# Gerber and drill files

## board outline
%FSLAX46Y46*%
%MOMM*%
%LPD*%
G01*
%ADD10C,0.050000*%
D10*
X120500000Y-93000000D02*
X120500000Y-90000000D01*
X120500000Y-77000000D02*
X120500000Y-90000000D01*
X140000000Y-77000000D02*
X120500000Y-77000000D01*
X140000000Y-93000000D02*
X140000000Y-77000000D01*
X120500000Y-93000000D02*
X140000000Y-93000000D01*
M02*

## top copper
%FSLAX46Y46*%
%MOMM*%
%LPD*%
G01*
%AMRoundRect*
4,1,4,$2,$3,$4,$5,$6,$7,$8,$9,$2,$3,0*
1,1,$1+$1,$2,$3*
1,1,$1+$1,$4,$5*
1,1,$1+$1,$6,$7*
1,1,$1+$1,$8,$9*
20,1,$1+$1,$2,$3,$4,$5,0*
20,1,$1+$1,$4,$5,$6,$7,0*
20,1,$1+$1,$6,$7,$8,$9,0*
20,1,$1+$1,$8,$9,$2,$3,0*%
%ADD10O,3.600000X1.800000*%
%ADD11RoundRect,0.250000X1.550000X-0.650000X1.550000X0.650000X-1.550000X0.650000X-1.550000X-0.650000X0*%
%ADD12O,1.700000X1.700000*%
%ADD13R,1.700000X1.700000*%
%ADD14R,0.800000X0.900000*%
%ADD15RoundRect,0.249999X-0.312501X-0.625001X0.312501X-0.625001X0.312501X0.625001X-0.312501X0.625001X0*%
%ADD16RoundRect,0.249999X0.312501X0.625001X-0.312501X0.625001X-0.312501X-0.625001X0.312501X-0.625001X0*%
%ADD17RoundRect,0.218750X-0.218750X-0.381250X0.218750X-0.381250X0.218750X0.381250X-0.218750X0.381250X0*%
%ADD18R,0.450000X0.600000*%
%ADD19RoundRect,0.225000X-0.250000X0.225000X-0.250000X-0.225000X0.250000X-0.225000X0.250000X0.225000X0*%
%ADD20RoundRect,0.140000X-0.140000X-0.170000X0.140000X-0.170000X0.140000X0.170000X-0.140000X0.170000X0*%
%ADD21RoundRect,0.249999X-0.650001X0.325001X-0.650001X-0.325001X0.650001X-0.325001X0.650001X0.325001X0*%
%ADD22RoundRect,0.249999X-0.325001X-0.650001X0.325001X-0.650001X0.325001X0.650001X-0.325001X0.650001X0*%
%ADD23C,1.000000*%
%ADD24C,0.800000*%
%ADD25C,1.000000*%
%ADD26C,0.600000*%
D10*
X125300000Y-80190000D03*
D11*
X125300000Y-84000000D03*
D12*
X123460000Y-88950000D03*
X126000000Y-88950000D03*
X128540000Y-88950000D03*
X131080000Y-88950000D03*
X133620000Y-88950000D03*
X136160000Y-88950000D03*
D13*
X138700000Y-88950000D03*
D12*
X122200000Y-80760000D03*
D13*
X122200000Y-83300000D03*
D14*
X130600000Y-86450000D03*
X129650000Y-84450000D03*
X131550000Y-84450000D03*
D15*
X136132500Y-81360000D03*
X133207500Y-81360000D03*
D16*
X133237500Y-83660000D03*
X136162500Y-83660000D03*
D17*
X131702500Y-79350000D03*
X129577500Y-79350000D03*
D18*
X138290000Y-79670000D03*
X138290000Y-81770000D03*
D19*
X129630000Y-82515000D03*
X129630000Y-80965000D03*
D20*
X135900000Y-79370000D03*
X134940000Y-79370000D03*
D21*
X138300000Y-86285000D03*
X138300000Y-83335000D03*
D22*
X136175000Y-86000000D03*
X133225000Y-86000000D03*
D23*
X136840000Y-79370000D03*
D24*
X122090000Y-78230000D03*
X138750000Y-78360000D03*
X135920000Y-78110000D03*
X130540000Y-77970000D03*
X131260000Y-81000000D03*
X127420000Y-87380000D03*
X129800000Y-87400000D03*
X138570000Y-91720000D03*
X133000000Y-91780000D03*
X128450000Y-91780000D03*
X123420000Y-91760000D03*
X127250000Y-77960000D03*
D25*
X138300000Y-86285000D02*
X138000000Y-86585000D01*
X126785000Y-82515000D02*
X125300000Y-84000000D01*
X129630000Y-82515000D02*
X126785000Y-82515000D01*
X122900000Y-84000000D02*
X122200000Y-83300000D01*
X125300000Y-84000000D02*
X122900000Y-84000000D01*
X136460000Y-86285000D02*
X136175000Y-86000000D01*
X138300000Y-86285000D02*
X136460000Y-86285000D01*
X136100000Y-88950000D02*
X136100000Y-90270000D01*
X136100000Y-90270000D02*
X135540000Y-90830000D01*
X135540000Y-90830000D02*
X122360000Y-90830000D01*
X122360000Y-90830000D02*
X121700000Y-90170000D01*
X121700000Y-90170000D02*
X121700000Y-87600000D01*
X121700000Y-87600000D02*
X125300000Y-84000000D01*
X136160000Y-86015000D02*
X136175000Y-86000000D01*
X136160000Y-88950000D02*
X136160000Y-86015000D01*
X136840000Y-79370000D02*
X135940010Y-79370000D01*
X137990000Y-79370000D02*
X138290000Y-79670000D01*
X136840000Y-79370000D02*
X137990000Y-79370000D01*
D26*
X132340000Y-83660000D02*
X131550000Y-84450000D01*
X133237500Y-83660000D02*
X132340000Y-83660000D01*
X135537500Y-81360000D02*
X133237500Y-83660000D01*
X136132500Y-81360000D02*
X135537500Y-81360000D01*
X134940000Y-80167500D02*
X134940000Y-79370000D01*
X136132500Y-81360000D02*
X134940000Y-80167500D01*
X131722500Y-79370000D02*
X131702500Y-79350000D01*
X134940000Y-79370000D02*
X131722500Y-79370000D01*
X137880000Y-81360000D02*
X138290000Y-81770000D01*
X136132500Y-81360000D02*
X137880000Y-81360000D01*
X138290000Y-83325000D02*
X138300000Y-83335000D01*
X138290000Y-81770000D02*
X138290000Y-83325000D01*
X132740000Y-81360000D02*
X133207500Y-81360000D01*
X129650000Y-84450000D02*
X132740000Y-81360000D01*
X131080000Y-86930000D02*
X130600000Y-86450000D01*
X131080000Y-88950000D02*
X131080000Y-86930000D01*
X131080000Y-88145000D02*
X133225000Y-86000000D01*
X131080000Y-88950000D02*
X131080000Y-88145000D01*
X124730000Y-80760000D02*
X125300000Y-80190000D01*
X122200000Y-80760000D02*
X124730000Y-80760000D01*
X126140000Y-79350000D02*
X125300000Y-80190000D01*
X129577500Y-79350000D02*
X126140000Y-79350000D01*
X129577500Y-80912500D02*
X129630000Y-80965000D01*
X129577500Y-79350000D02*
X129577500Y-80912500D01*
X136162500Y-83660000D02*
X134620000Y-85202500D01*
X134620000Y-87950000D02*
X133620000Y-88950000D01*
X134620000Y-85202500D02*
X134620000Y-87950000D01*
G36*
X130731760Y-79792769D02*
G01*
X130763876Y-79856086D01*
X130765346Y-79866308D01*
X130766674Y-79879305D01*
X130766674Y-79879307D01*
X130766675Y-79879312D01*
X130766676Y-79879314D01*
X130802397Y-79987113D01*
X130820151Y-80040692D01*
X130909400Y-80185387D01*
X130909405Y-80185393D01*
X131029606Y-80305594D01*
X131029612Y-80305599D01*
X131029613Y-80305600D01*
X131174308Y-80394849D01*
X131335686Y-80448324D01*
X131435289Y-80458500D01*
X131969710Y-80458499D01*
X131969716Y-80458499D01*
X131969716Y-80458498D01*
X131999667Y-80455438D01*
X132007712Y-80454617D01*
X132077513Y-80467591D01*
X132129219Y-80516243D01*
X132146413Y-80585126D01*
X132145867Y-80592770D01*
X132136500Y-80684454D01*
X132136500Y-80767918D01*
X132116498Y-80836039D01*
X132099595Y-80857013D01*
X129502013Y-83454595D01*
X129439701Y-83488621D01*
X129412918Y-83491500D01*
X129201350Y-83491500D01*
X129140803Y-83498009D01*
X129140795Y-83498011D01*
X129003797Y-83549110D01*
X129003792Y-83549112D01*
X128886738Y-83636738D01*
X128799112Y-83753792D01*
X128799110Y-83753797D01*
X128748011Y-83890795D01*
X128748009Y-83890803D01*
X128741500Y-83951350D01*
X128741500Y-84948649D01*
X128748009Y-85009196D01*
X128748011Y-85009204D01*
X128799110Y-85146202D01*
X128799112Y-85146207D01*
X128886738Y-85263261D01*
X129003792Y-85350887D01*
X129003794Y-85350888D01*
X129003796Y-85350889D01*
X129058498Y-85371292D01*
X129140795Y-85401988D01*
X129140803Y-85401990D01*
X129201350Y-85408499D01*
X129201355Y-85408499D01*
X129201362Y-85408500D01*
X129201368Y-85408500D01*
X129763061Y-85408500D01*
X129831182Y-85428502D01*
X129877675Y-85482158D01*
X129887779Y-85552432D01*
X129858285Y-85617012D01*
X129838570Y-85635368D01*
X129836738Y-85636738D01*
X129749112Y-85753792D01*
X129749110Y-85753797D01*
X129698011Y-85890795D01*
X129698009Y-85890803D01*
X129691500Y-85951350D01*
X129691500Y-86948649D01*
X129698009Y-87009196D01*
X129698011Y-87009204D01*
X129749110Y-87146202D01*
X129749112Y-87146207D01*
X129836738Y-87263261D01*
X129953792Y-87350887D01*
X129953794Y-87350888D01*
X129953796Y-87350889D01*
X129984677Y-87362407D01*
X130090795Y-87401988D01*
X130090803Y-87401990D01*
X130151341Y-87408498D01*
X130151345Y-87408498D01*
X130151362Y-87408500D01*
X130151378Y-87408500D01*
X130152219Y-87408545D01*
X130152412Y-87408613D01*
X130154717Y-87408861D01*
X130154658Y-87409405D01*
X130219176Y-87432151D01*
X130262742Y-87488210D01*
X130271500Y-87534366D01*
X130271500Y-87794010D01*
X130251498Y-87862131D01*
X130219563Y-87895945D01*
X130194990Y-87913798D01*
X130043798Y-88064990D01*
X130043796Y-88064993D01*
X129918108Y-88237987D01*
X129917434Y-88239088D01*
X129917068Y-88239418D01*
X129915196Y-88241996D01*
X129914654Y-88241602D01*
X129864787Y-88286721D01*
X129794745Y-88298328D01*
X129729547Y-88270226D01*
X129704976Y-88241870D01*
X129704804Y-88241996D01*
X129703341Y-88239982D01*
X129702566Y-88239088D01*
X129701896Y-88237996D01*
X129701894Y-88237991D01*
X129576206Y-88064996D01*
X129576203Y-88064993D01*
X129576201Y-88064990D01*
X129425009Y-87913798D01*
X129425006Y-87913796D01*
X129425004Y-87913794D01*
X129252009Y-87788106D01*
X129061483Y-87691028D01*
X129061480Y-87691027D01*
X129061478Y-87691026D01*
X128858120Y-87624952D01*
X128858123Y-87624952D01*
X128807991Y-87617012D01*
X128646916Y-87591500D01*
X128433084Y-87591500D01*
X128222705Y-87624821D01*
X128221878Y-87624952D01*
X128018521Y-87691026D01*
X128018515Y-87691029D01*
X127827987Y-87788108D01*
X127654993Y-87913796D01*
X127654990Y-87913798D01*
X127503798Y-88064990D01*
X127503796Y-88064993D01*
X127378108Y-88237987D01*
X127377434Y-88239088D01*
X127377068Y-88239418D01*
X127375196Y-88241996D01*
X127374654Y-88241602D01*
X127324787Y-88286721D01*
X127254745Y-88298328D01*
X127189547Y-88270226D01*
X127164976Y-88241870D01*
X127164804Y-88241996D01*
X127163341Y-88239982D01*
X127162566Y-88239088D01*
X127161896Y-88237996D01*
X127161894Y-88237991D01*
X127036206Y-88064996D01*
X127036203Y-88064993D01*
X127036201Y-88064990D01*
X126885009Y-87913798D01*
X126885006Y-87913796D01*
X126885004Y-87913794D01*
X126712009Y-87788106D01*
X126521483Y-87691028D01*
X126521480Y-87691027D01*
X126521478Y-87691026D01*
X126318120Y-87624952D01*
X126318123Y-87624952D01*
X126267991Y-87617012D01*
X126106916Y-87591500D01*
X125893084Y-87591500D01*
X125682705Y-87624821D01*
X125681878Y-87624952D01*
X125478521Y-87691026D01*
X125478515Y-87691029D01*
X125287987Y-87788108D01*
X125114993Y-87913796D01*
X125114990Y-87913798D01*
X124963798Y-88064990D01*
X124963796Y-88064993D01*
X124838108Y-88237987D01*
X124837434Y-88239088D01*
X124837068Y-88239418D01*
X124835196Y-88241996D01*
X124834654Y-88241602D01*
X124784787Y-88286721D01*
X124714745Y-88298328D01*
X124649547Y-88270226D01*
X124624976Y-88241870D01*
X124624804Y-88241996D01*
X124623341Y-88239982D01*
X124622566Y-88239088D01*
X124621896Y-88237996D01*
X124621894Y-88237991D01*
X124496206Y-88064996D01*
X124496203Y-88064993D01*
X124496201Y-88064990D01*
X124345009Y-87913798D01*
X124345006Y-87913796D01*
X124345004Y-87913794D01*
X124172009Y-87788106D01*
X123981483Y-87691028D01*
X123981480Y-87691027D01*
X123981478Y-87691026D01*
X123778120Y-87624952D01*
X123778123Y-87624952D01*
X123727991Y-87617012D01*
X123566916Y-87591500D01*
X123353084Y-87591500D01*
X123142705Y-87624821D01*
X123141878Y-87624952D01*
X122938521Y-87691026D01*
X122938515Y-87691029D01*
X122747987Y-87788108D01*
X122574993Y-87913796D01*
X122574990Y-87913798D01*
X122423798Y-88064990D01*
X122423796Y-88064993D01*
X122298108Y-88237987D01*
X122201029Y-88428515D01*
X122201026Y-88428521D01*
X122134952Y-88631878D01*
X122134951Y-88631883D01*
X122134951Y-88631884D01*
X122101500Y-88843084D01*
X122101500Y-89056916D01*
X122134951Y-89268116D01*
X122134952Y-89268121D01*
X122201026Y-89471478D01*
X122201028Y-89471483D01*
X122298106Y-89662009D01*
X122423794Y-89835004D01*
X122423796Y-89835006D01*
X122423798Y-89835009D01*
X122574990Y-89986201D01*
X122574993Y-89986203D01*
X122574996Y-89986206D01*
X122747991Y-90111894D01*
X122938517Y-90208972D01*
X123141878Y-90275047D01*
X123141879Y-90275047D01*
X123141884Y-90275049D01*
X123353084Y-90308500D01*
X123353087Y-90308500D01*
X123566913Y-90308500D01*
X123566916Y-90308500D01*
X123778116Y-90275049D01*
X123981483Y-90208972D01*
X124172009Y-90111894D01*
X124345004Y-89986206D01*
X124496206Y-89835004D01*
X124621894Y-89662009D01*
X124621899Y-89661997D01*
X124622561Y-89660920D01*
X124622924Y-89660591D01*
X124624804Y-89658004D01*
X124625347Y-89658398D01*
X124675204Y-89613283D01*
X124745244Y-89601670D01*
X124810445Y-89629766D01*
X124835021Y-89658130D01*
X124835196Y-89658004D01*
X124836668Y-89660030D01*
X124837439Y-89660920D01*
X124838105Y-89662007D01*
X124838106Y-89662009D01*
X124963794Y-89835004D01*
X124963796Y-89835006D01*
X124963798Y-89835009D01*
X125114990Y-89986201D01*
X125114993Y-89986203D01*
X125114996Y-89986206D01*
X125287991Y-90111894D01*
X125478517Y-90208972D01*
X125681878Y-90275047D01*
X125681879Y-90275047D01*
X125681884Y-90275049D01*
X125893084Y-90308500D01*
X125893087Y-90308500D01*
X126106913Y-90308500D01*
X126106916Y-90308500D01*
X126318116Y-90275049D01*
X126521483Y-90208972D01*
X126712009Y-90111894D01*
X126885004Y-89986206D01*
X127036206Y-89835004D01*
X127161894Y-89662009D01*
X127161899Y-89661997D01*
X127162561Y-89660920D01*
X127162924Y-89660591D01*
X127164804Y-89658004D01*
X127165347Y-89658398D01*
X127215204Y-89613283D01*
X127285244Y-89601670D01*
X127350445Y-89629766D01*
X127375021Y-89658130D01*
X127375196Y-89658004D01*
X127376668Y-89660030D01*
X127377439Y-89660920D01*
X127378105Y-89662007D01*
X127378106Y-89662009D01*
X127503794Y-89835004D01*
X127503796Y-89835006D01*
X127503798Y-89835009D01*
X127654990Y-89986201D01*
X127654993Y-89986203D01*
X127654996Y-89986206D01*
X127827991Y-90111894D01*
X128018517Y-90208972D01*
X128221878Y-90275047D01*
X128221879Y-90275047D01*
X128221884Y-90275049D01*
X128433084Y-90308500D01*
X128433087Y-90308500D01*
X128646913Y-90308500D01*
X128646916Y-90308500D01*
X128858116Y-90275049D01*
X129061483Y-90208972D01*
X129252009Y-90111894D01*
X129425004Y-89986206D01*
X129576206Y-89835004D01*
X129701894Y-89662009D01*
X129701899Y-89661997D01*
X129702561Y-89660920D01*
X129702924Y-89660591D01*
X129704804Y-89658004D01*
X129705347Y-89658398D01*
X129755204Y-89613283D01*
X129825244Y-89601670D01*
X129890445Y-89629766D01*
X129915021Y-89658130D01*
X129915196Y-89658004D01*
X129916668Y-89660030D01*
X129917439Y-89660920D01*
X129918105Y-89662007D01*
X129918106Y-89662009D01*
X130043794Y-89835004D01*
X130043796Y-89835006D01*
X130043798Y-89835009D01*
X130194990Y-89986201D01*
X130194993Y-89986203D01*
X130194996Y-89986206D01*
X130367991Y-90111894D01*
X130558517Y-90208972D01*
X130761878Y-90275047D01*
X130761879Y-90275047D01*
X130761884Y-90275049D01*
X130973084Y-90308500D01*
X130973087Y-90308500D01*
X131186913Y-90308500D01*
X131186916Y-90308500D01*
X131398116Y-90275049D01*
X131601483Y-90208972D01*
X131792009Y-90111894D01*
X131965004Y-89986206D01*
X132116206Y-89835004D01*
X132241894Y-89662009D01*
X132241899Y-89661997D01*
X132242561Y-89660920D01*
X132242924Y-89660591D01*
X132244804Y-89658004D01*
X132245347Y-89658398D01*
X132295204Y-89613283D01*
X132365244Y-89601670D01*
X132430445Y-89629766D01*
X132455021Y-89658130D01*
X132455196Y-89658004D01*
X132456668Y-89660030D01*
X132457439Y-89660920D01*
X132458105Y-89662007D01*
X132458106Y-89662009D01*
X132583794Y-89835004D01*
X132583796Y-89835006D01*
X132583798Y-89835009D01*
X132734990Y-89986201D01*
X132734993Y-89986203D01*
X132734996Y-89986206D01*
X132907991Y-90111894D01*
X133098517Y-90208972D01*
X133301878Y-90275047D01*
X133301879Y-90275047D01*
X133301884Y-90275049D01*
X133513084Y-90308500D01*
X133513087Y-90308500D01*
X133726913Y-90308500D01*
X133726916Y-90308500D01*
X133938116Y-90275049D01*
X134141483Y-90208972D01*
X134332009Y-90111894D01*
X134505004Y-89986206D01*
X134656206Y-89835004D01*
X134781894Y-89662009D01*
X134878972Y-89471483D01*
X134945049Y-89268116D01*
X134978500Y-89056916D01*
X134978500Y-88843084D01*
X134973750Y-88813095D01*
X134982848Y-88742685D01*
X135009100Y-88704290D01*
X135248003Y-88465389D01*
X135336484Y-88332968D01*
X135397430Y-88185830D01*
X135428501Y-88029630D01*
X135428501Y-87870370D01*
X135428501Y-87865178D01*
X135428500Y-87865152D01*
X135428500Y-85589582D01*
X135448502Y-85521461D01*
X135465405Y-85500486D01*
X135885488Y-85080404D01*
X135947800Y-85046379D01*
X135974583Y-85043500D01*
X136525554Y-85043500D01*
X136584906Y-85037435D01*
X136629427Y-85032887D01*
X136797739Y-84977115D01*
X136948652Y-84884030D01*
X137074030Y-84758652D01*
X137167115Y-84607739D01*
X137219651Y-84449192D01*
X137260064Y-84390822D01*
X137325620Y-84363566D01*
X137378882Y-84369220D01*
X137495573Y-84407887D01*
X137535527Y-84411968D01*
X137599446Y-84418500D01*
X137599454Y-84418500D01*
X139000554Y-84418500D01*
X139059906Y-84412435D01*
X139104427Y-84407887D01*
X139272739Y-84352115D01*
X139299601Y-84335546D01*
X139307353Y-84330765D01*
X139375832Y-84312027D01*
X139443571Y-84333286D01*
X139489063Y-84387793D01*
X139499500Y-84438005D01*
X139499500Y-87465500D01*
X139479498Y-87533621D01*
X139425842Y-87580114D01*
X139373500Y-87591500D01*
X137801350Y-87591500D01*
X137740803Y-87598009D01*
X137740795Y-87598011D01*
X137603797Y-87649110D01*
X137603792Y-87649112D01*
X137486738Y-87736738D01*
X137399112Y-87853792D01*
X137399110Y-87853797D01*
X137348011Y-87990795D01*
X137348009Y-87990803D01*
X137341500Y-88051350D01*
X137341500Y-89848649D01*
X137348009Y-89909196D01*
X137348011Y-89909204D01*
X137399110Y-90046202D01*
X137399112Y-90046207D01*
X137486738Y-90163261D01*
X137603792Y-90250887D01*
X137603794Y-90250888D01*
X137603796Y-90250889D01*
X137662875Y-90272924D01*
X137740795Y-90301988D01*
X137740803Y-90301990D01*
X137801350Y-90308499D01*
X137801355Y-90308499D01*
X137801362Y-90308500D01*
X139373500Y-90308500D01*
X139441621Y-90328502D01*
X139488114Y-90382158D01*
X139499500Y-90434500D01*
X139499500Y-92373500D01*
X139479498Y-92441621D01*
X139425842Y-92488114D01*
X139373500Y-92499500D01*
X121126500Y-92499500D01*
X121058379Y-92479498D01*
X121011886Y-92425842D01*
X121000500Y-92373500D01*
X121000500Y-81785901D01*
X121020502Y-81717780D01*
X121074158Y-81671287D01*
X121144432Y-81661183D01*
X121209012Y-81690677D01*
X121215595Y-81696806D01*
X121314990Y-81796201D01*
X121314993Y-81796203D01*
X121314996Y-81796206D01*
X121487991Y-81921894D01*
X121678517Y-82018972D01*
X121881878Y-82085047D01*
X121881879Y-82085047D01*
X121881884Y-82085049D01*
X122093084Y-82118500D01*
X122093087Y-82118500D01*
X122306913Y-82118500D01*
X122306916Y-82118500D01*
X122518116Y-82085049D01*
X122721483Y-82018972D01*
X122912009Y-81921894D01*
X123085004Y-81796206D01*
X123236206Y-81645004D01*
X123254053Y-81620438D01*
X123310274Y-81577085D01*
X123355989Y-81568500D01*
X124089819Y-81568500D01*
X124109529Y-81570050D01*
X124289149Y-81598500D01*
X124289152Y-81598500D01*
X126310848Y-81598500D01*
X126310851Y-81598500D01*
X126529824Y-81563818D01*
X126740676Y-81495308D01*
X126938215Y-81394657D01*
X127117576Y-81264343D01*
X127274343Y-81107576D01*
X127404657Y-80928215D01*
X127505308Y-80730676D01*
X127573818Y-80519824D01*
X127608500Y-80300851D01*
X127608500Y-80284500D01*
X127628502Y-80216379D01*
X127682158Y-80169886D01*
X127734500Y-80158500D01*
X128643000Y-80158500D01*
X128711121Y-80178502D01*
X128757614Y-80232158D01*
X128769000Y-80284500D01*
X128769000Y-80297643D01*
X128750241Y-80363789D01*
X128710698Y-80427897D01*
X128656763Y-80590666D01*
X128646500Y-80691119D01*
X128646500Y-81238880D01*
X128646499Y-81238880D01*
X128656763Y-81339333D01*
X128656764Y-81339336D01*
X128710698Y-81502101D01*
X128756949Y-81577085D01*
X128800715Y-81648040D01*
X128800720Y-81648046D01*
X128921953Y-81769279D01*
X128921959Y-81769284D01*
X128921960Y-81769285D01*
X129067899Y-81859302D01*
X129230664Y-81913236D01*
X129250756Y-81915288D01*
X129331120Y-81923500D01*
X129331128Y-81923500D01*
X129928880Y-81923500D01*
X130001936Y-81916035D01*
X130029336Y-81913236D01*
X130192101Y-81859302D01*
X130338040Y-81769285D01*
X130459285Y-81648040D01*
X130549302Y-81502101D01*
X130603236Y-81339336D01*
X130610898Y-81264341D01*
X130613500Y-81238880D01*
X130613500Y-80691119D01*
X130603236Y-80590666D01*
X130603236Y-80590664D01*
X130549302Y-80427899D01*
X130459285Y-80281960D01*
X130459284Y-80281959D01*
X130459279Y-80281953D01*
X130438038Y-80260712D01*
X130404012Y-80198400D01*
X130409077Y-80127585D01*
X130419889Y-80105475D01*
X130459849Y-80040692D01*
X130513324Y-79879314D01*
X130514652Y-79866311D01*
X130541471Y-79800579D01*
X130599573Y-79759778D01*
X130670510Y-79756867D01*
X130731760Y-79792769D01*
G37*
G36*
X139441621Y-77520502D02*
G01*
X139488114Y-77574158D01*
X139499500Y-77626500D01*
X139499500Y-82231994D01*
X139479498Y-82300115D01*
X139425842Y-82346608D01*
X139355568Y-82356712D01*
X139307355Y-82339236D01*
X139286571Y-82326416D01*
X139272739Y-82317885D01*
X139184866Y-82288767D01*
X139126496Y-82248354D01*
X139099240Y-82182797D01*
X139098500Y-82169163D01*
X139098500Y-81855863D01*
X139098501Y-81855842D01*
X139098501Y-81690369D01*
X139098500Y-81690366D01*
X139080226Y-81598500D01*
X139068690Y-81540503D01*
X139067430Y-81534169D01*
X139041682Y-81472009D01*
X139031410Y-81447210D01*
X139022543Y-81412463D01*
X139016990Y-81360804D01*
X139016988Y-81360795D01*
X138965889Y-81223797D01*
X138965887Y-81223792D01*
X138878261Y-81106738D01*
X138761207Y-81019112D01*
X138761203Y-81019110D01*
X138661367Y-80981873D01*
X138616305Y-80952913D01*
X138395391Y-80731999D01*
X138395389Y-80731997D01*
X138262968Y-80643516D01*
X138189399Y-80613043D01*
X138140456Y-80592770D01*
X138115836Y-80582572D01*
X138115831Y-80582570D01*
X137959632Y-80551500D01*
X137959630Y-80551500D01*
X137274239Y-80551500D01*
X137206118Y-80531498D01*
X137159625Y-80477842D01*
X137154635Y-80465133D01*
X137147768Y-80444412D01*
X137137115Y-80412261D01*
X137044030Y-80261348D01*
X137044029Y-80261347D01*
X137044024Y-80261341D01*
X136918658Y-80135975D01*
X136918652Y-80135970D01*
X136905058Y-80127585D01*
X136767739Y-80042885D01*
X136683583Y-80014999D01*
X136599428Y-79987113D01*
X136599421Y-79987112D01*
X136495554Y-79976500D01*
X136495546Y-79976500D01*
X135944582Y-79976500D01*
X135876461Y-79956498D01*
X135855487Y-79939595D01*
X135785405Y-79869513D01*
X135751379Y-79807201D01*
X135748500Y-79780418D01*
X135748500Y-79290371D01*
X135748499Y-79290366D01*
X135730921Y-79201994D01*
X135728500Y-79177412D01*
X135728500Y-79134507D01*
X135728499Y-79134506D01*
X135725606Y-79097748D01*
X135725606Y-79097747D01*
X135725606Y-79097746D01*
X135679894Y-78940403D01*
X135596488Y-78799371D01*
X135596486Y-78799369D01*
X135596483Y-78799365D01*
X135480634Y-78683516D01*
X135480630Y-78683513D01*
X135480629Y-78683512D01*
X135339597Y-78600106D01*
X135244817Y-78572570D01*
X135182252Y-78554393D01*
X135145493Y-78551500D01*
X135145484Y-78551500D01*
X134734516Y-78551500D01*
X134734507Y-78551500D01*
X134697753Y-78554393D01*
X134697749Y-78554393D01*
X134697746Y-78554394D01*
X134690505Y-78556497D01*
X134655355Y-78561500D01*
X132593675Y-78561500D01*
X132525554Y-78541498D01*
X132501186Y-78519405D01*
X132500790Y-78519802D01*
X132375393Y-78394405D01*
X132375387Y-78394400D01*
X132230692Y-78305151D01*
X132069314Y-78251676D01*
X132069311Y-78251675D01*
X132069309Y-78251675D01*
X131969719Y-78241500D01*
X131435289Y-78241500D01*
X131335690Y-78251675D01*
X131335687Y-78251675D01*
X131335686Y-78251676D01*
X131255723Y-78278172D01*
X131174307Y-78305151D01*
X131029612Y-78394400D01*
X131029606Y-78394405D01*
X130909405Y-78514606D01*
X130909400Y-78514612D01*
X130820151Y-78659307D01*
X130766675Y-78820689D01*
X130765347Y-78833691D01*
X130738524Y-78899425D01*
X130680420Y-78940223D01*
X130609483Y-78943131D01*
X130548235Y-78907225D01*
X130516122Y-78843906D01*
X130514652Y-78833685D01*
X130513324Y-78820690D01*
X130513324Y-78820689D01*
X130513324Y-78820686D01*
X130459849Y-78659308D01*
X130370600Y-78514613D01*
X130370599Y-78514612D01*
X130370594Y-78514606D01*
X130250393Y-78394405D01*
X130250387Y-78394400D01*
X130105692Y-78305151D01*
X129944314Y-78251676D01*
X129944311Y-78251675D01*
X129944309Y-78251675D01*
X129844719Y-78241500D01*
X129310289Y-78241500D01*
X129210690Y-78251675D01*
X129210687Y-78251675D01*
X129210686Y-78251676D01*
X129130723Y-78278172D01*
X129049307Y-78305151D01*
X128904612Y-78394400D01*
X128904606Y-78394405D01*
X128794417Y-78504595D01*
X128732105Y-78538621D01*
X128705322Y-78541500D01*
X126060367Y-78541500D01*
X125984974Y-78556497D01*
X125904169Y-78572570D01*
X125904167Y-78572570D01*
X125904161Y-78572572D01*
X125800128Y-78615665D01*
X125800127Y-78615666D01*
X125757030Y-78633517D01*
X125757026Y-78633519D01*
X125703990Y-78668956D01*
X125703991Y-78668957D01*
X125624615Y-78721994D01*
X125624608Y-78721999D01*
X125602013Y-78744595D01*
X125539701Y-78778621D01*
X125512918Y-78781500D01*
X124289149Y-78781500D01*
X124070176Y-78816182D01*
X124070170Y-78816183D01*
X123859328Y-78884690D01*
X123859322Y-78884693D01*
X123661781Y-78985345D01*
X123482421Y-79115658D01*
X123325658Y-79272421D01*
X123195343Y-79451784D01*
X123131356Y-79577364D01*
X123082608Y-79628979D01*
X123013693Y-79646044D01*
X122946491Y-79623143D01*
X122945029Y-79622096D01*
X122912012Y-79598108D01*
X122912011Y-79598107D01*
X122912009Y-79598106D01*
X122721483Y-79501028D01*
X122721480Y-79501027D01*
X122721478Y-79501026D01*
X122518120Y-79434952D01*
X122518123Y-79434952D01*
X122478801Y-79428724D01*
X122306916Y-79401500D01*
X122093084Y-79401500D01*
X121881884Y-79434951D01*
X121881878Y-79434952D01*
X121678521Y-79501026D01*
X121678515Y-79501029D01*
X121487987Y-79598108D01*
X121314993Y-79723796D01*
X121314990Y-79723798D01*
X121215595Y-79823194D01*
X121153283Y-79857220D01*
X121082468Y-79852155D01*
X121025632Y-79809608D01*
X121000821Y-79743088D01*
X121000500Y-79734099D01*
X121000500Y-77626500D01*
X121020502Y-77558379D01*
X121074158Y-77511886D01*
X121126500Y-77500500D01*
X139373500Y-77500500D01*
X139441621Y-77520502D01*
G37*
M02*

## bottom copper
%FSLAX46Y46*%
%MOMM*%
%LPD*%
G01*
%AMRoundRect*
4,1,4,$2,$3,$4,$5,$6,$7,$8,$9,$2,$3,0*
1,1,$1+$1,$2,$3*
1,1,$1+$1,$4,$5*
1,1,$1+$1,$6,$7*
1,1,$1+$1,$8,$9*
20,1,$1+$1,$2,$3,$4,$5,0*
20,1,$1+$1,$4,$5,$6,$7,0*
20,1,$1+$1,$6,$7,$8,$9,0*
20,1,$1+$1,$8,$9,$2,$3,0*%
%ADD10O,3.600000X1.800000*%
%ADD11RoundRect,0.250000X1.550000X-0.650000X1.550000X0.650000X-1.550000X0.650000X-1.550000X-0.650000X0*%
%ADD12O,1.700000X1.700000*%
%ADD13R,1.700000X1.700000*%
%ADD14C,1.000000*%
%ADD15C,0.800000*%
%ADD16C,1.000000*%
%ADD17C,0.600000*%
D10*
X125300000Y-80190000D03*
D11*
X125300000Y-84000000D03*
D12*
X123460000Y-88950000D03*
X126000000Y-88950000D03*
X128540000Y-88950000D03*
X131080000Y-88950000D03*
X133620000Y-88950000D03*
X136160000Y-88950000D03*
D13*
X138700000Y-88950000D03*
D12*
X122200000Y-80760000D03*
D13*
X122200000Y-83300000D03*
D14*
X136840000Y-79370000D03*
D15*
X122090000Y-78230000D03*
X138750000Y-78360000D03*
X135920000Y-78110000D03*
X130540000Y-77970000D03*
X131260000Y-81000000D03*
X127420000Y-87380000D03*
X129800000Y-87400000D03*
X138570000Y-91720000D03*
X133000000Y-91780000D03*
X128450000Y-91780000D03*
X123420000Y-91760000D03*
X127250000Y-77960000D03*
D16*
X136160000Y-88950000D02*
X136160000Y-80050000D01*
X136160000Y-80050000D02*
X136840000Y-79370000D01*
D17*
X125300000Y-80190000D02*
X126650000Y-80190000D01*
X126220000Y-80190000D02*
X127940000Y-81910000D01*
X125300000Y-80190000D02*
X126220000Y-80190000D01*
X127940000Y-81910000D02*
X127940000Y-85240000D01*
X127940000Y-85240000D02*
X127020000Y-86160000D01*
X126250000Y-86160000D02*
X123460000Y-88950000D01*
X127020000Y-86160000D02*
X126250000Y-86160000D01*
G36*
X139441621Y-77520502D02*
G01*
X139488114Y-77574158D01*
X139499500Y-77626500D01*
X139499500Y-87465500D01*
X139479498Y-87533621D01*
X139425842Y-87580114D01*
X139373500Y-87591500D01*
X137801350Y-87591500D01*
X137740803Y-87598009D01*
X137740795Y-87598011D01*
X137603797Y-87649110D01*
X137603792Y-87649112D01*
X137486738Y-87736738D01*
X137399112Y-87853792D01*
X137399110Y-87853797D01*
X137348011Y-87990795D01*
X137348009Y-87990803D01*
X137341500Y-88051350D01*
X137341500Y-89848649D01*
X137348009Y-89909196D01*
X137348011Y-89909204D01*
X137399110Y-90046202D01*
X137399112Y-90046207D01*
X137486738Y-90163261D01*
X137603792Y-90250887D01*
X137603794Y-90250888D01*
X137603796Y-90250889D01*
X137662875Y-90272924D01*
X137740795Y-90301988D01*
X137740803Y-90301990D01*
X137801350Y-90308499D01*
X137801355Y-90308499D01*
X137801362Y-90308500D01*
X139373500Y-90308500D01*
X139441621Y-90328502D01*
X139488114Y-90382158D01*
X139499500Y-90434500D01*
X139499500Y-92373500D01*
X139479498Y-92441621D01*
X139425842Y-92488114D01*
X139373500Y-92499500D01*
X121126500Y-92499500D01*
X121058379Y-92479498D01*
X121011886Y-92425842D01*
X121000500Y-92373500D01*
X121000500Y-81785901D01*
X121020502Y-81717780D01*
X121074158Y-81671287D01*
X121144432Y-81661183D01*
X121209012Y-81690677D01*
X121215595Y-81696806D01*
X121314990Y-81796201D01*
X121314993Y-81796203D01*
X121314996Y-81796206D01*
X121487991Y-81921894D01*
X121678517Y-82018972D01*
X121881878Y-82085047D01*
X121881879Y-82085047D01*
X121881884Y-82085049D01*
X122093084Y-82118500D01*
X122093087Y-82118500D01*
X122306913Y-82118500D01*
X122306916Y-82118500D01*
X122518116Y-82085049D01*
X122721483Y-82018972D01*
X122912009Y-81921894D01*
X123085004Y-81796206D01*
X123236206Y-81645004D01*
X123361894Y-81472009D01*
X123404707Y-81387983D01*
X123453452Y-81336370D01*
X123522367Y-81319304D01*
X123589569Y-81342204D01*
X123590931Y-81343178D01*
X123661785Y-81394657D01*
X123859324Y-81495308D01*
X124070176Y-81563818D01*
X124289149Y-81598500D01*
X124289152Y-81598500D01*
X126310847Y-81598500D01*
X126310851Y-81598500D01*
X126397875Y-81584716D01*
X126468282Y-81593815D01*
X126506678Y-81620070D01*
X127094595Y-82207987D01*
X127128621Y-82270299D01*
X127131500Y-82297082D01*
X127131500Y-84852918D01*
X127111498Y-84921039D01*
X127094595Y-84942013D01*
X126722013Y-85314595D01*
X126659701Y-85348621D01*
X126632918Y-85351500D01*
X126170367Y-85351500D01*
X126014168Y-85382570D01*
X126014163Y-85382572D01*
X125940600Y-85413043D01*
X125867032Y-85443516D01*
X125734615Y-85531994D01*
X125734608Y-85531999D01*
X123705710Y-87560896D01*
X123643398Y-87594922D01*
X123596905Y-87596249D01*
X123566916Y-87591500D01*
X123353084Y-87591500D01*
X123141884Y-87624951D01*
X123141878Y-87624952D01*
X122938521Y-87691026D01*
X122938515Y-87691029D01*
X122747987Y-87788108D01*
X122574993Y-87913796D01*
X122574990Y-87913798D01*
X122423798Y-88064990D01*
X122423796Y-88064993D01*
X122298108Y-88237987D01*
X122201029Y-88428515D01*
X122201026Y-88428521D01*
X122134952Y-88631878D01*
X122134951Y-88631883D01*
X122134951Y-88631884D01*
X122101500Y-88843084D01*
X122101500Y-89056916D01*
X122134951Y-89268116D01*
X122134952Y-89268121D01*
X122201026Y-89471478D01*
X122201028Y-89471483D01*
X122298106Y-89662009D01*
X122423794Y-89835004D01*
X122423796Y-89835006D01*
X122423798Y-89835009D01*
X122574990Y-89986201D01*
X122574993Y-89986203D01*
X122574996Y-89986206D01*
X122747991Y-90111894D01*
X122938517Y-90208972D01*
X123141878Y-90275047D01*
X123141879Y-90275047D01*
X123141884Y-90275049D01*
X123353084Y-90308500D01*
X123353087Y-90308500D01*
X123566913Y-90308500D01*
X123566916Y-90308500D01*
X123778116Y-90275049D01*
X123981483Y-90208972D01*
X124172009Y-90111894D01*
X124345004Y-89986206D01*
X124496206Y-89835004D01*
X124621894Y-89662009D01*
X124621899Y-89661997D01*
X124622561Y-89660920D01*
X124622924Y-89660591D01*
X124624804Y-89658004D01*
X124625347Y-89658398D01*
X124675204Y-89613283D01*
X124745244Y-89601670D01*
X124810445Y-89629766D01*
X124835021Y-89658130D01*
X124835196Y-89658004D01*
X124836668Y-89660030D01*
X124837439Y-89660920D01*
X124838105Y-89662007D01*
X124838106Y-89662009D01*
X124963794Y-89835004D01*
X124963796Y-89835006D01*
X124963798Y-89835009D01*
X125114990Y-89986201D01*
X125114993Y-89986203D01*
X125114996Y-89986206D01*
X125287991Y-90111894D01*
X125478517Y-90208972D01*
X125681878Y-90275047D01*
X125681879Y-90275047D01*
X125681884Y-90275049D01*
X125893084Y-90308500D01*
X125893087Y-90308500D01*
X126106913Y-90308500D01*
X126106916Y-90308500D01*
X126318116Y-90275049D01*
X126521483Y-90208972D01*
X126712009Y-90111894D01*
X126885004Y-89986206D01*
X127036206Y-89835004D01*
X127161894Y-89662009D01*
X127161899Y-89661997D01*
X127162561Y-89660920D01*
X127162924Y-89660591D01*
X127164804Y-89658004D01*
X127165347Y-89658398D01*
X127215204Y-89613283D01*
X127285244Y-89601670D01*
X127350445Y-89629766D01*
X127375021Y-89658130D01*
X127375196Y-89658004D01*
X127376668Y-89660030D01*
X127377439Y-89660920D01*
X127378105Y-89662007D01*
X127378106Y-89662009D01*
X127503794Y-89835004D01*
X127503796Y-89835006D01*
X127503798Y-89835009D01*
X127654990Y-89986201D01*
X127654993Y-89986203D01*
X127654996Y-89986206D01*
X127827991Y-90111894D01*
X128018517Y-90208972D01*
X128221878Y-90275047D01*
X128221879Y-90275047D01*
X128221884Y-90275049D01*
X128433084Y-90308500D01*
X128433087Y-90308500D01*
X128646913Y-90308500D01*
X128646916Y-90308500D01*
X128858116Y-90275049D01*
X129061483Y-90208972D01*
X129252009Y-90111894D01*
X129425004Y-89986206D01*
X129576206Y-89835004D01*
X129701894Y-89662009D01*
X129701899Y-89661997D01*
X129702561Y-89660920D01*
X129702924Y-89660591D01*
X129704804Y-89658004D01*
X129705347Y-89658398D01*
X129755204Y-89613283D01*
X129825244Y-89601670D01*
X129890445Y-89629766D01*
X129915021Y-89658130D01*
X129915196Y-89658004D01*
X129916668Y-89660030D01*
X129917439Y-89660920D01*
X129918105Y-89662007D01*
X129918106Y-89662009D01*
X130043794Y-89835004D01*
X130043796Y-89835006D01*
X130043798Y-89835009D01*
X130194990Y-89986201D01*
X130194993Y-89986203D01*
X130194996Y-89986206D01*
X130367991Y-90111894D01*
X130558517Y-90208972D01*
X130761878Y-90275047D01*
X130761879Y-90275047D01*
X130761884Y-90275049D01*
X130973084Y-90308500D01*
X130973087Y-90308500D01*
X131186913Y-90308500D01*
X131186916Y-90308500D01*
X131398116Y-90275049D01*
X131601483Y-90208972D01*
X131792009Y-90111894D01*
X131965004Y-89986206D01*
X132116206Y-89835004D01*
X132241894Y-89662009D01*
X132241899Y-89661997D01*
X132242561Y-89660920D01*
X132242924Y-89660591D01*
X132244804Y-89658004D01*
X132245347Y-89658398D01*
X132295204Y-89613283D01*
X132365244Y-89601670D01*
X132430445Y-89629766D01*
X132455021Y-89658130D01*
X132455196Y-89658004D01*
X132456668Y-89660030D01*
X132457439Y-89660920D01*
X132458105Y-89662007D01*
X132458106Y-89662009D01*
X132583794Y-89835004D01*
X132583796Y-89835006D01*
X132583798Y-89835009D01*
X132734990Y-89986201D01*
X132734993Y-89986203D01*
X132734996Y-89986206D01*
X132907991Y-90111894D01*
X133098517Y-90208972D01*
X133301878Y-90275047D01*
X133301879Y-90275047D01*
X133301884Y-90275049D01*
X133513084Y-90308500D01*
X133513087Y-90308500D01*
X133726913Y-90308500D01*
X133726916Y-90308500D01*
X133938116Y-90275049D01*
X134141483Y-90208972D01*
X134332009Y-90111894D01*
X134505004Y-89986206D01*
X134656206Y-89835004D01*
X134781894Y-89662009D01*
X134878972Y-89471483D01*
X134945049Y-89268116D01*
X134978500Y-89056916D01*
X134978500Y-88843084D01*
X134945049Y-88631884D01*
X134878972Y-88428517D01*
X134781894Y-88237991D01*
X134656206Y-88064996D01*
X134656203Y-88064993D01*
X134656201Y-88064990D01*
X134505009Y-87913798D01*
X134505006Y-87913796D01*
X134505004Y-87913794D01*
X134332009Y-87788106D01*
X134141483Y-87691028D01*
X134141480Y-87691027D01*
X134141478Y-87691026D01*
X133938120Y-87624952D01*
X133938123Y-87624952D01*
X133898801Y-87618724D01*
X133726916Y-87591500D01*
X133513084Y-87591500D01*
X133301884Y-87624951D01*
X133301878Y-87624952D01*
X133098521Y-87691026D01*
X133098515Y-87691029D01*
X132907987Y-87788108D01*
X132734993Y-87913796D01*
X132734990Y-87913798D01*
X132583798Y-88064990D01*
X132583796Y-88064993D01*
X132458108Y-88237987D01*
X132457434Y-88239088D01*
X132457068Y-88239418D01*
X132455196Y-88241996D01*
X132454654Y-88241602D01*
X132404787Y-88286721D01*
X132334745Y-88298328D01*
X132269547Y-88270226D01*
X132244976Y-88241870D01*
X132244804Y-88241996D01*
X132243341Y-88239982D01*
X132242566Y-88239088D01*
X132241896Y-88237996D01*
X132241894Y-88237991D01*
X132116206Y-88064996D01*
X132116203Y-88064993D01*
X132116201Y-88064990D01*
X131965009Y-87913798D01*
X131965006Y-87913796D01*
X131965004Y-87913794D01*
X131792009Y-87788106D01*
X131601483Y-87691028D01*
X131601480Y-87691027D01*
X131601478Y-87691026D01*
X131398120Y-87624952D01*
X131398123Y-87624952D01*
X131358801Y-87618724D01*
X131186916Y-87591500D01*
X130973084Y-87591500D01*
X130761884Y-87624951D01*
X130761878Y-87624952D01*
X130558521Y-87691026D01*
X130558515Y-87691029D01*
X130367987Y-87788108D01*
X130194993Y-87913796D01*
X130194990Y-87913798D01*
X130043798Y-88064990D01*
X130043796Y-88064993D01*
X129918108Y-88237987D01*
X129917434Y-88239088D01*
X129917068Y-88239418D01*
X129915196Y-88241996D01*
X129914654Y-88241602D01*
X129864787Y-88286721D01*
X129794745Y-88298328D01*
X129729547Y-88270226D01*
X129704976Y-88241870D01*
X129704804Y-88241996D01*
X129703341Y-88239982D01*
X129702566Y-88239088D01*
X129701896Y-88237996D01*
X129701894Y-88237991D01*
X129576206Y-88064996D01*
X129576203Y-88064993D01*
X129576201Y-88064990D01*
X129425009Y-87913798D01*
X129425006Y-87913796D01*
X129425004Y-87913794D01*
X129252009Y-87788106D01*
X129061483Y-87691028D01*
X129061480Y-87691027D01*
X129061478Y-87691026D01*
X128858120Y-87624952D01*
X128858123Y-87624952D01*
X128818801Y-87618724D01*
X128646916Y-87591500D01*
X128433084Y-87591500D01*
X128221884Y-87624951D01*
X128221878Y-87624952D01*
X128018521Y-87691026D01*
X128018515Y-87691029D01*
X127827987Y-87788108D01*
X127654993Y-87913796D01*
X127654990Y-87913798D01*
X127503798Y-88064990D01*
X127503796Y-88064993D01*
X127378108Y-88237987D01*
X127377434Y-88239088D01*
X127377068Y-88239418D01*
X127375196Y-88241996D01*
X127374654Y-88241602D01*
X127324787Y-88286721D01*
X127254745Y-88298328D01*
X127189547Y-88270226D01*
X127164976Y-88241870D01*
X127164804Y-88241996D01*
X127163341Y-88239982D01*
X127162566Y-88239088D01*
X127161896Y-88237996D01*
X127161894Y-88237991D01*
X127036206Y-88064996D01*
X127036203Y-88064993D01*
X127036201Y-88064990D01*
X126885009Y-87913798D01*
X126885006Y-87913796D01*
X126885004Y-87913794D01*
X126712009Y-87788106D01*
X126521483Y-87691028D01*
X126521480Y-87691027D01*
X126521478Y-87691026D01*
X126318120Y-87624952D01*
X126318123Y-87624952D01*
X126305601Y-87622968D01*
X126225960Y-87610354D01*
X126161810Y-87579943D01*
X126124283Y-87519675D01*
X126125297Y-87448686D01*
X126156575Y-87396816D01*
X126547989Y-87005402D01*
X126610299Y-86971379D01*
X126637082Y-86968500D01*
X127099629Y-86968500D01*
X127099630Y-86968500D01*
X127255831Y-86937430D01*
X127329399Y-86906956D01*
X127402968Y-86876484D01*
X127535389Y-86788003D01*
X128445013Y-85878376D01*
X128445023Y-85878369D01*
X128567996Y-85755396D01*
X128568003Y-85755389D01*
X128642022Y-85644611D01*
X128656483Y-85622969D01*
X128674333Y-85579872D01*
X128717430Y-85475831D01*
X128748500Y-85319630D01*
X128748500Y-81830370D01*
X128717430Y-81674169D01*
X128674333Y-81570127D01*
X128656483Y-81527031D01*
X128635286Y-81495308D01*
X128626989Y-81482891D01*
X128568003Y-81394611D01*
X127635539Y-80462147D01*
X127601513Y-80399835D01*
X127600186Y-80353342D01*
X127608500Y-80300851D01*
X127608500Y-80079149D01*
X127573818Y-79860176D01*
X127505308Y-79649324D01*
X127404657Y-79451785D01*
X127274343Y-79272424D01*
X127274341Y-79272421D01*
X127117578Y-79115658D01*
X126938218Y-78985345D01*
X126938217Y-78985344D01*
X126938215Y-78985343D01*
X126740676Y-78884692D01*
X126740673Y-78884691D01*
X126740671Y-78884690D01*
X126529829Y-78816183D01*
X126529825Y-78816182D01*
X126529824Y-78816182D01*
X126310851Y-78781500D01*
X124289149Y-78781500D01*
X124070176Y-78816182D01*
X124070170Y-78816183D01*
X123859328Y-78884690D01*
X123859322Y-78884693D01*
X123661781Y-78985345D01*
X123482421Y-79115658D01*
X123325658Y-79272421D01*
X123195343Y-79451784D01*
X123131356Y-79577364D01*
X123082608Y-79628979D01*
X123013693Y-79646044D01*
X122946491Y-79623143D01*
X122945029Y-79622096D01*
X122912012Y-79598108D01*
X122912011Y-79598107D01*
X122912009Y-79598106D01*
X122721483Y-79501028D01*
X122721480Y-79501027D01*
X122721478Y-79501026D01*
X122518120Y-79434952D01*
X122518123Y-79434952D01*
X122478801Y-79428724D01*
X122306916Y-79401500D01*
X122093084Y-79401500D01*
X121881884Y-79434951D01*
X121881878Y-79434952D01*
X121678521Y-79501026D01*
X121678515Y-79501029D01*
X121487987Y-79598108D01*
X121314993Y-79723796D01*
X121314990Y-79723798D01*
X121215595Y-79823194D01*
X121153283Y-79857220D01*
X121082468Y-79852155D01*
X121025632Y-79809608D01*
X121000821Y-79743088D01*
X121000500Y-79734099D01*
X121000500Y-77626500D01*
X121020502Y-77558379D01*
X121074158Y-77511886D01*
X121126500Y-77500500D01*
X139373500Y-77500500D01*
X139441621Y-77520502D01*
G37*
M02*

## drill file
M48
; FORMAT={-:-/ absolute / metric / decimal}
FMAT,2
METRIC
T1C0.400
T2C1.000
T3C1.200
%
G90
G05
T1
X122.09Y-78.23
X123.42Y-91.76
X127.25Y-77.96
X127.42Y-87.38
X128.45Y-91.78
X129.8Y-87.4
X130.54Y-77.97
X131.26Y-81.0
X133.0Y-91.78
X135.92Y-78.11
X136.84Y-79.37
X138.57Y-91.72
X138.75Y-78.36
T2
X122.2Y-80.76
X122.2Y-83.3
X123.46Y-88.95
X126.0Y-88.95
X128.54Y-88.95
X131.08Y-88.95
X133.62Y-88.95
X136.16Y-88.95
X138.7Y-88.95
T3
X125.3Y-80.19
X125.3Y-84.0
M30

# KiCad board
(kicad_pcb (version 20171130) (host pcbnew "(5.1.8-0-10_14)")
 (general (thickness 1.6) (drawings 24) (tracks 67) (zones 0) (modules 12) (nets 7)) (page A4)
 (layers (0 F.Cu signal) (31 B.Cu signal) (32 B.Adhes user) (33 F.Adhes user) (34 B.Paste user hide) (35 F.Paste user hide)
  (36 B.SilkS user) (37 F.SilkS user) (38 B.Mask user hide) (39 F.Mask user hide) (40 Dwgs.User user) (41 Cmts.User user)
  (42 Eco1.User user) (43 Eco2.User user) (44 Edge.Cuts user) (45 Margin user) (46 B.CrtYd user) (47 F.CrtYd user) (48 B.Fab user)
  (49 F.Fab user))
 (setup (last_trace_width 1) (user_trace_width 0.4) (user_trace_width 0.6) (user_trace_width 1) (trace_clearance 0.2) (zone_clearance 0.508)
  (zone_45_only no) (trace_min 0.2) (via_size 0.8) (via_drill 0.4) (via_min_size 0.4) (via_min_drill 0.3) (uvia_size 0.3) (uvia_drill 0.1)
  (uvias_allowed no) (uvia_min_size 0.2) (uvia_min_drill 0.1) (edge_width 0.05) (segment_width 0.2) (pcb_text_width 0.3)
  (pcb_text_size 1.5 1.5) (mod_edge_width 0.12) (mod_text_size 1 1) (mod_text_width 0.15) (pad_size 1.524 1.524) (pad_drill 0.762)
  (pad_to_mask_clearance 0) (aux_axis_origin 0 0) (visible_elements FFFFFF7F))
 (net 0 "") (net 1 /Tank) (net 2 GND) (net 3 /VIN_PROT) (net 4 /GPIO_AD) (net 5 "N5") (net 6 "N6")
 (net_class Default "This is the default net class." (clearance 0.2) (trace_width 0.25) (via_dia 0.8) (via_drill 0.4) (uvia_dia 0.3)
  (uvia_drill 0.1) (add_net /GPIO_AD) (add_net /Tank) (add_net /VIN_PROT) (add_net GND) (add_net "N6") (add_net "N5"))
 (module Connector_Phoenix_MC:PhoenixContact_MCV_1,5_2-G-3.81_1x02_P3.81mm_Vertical (layer F.Cu) (at 125.3 84 90)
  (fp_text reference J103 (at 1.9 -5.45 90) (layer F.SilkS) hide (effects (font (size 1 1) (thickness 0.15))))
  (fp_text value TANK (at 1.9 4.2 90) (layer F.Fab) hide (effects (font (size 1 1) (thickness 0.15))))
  (pad 2 thru_hole oval (at 3.81 0 90) (size 1.8 3.6) (drill 1.2) (layers *.Cu *.Mask) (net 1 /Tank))
  (pad 1 thru_hole roundrect (at 0 0 90) (size 1.8 3.6) (drill 1.2) (layers *.Cu *.Mask) (roundrect_rratio 0.138889) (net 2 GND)))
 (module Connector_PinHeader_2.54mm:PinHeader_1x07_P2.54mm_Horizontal (layer F.Cu) (at 138.7 88.95 270)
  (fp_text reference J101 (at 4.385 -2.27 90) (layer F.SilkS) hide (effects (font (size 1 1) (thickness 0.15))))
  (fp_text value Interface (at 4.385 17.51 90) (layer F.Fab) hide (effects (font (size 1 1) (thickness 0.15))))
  (pad 7 thru_hole oval (at 0 15.24 270) (size 1.7 1.7) (drill 1) (layers *.Cu *.Mask) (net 1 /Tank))
  (pad 6 thru_hole oval (at 0 12.7 270) (size 1.7 1.7) (drill 1) (layers *.Cu *.Mask))
  (pad 5 thru_hole oval (at 0 10.16 270) (size 1.7 1.7) (drill 1) (layers *.Cu *.Mask))
  (pad 4 thru_hole oval (at 0 7.62 270) (size 1.7 1.7) (drill 1) (layers *.Cu *.Mask) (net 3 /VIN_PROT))
  (pad 3 thru_hole oval (at 0 5.08 270) (size 1.7 1.7) (drill 1) (layers *.Cu *.Mask) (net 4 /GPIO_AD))
  (pad 2 thru_hole oval (at 0 2.54 270) (size 1.7 1.7) (drill 1) (layers *.Cu *.Mask) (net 2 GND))
  (pad 1 thru_hole rect (at 0 0 270) (size 1.7 1.7) (drill 1) (layers *.Cu *.Mask)))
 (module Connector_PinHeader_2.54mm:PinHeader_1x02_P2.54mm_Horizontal (layer F.Cu) (at 122.2 83.3 180)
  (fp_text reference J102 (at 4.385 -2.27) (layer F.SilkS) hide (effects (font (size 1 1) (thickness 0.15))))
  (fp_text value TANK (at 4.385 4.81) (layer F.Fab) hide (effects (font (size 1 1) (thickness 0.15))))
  (pad 2 thru_hole oval (at 0 2.54 180) (size 1.7 1.7) (drill 1) (layers *.Cu *.Mask) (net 1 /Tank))
  (pad 1 thru_hole rect (at 0 0 180) (size 1.7 1.7) (drill 1) (layers *.Cu *.Mask) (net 2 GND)))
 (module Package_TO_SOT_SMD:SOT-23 (layer F.Cu) (at 130.6 85.45 270)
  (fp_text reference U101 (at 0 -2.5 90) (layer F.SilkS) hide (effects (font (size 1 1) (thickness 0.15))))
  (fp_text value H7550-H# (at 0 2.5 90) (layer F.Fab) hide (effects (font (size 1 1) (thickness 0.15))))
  (pad 3 smd rect (at 1 0 270) (size 0.9 0.8) (layers F.Cu F.Paste F.Mask) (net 3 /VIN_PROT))
  (pad 2 smd rect (at -1 0.95 270) (size 0.9 0.8) (layers F.Cu F.Paste F.Mask) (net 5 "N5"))
  (pad 1 smd rect (at -1 -0.95 270) (size 0.9 0.8) (layers F.Cu F.Paste F.Mask) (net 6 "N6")))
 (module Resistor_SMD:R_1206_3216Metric (layer F.Cu) (at 134.67 81.36)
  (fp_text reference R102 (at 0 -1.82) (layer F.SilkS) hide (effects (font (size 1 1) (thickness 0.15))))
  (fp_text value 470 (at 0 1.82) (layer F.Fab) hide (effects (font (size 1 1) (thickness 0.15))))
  (pad 2 smd roundrect (at 1.4625 0) (size 1.125 1.75) (layers F.Cu F.Paste F.Mask) (roundrect_rratio 0.2222213333333333) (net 6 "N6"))
  (pad 1 smd roundrect (at -1.4625 0) (size 1.125 1.75) (layers F.Cu F.Paste F.Mask) (roundrect_rratio 0.2222213333333333) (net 5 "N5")))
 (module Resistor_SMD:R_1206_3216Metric (layer F.Cu) (at 134.7 83.66 180)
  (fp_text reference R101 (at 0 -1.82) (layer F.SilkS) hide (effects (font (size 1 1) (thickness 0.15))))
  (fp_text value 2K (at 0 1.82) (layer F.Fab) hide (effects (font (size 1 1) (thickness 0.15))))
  (pad 2 smd roundrect (at 1.4625 0 180) (size 1.125 1.75) (layers F.Cu F.Paste F.Mask) (roundrect_rratio 0.2222213333333333) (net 6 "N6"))
  (pad 1 smd roundrect (at -1.4625 0 180) (size 1.125 1.75) (layers F.Cu F.Paste F.Mask) (roundrect_rratio 0.2222213333333333)
   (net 4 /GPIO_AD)))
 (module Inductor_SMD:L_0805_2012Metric (layer F.Cu) (at 130.64 79.35)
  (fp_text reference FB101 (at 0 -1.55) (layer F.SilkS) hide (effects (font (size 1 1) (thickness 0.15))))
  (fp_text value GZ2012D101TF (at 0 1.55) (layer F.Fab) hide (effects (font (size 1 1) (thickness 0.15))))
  (pad 2 smd roundrect (at 1.0625 0) (size 0.875 1.2) (layers F.Cu F.Paste F.Mask) (roundrect_rratio 0.25) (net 6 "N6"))
  (pad 1 smd roundrect (at -1.0625 0) (size 0.875 1.2) (layers F.Cu F.Paste F.Mask) (roundrect_rratio 0.25) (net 1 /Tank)))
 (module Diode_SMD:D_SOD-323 (layer F.Cu) (at 138.29 80.72 90)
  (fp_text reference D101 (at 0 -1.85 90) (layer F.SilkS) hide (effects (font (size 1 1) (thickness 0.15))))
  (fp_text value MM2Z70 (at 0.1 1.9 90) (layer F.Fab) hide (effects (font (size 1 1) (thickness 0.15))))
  (pad 2 smd rect (at 1.05 0 90) (size 0.6 0.45) (layers F.Cu F.Paste F.Mask) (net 2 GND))
  (pad 1 smd rect (at -1.05 0 90) (size 0.6 0.45) (layers F.Cu F.Paste F.Mask) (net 6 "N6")))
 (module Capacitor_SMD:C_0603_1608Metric (layer F.Cu) (at 129.63 81.74 270)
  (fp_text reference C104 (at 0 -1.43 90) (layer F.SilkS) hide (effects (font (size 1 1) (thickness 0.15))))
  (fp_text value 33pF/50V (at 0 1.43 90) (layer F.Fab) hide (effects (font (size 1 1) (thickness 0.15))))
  (pad 2 smd roundrect (at 0.775 0 270) (size 0.9 0.95) (layers F.Cu F.Paste F.Mask) (roundrect_rratio 0.25) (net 2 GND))
  (pad 1 smd roundrect (at -0.775 0 270) (size 0.9 0.95) (layers F.Cu F.Paste F.Mask) (roundrect_rratio 0.25) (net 1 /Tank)))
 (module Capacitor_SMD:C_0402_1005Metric (layer F.Cu) (at 135.42 79.37)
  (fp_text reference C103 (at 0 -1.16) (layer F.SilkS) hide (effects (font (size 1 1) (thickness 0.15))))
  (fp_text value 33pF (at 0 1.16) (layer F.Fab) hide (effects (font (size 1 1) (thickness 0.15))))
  (pad 2 smd roundrect (at 0.48 0) (size 0.56 0.62) (layers F.Cu F.Paste F.Mask) (roundrect_rratio 0.25) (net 2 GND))
  (pad 1 smd roundrect (at -0.48 0) (size 0.56 0.62) (layers F.Cu F.Paste F.Mask) (roundrect_rratio 0.25) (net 6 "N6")))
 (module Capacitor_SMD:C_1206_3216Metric (layer F.Cu) (at 138.3 84.81 270)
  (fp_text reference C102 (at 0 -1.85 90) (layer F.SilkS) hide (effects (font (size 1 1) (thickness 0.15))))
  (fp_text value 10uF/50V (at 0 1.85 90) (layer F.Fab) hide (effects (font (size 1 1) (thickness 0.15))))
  (pad 2 smd roundrect (at 1.475 0 270) (size 1.15 1.8) (layers F.Cu F.Paste F.Mask) (roundrect_rratio 0.2173904347826087) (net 2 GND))
  (pad 1 smd roundrect (at -1.475 0 270) (size 1.15 1.8) (layers F.Cu F.Paste F.Mask) (roundrect_rratio 0.2173904347826087) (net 6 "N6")))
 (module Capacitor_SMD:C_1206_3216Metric (layer F.Cu) (at 134.7 86)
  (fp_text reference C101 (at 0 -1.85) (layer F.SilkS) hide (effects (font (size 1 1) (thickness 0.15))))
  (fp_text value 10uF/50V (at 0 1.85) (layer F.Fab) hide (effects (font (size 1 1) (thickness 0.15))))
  (pad 2 smd roundrect (at 1.475 0) (size 1.15 1.8) (layers F.Cu F.Paste F.Mask) (roundrect_rratio 0.2173904347826087) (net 2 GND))
  (pad 1 smd roundrect (at -1.475 0) (size 1.15 1.8) (layers F.Cu F.Paste F.Mask) (roundrect_rratio 0.2173904347826087) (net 3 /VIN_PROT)))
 (gr_line (start 120.5 93) (end 120.5 90) (layer Edge.Cuts) (width 0.05))
 (gr_line (start 120.5 77) (end 120.5 90) (layer Edge.Cuts) (width 0.05))
 (gr_line (start 140 77) (end 120.5 77) (layer Edge.Cuts) (width 0.05))
 (gr_line (start 140 93) (end 140 77) (layer Edge.Cuts) (width 0.05))
 (gr_line (start 120.5 93) (end 140 93) (layer Edge.Cuts) (width 0.05))
 (segment (start 138.3 86.285) (end 138 86.585) (width 1) (layer F.Cu) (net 2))
 (segment (start 126.785 82.515) (end 125.3 84) (width 1) (layer F.Cu) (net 2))
 (segment (start 129.63 82.515) (end 126.785 82.515) (width 1) (layer F.Cu) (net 2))
 (segment (start 122.9 84) (end 122.2 83.3) (width 1) (layer F.Cu) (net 2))
 (segment (start 125.3 84) (end 122.9 84) (width 1) (layer F.Cu) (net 2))
 (segment (start 136.46 86.285) (end 136.175 86) (width 1) (layer F.Cu) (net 2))
 (segment (start 138.3 86.285) (end 136.46 86.285) (width 1) (layer F.Cu) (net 2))
 (segment (start 136.1 88.95) (end 136.1 90.27) (width 1) (layer F.Cu) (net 2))
 (segment (start 136.1 90.27) (end 135.54 90.83) (width 1) (layer F.Cu) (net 2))
 (segment (start 135.54 90.83) (end 122.36 90.83) (width 1) (layer F.Cu) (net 2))
 (segment (start 122.36 90.83) (end 121.7 90.17) (width 1) (layer F.Cu) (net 2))
 (segment (start 121.7 90.17) (end 121.7 87.6) (width 1) (layer F.Cu) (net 2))
 (segment (start 121.7 87.6) (end 125.3 84) (width 1) (layer F.Cu) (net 2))
 (segment (start 136.16 86.015) (end 136.175 86) (width 1) (layer F.Cu) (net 2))
 (segment (start 136.16 88.95) (end 136.16 86.015) (width 1) (layer F.Cu) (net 2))
 (segment (start 136.16 88.95) (end 136.16 80.05) (width 1) (layer B.Cu) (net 2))
 (via (at 136.84 79.37) (size 1) (drill 0.4) (layers F.Cu B.Cu) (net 2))
 (segment (start 136.16 80.05) (end 136.84 79.37) (width 1) (layer B.Cu) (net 2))
 (segment (start 136.84 79.37) (end 135.94001 79.37) (width 1) (layer F.Cu) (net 2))
 (segment (start 137.99 79.37) (end 138.29 79.67) (width 1) (layer F.Cu) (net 2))
 (segment (start 136.84 79.37) (end 137.99 79.37) (width 1) (layer F.Cu) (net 2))
 (via (at 122.09 78.23) (size 0.8) (drill 0.4) (layers F.Cu B.Cu) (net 2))
 (via (at 138.75 78.36) (size 0.8) (drill 0.4) (layers F.Cu B.Cu) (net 2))
 (via (at 135.92 78.11) (size 0.8) (drill 0.4) (layers F.Cu B.Cu) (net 2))
 (via (at 130.54 77.97) (size 0.8) (drill 0.4) (layers F.Cu B.Cu) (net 2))
 (via (at 131.26 81) (size 0.8) (drill 0.4) (layers F.Cu B.Cu) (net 2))
 (via (at 127.42 87.38) (size 0.8) (drill 0.4) (layers F.Cu B.Cu) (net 2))
 (via (at 129.8 87.4) (size 0.8) (drill 0.4) (layers F.Cu B.Cu) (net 2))
 (via (at 138.57 91.72) (size 0.8) (drill 0.4) (layers F.Cu B.Cu) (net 2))
 (via (at 133 91.78) (size 0.8) (drill 0.4) (layers F.Cu B.Cu) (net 2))
 (via (at 128.45 91.78) (size 0.8) (drill 0.4) (layers F.Cu B.Cu) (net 2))
 (via (at 123.42 91.76) (size 0.8) (drill 0.4) (layers F.Cu B.Cu) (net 2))
 (via (at 127.25 77.96) (size 0.8) (drill 0.4) (layers F.Cu B.Cu) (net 2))
 (segment (start 132.34 83.66) (end 131.55 84.45) (width 0.6) (layer F.Cu) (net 6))
 (segment (start 133.2375 83.66) (end 132.34 83.66) (width 0.6) (layer F.Cu) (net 6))
 (segment (start 135.5375 81.36) (end 133.2375 83.66) (width 0.6) (layer F.Cu) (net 6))
 (segment (start 136.1325 81.36) (end 135.5375 81.36) (width 0.6) (layer F.Cu) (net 6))
 (segment (start 134.94 80.1675) (end 134.94 79.37) (width 0.6) (layer F.Cu) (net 6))
 (segment (start 136.1325 81.36) (end 134.94 80.1675) (width 0.6) (layer F.Cu) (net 6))
 (segment (start 131.7225 79.37) (end 131.7025 79.35) (width 0.6) (layer F.Cu) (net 6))
 (segment (start 134.94 79.37) (end 131.7225 79.37) (width 0.6) (layer F.Cu) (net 6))
 (segment (start 137.88 81.36) (end 138.29 81.77) (width 0.6) (layer F.Cu) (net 6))
 (segment (start 136.1325 81.36) (end 137.88 81.36) (width 0.6) (layer F.Cu) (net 6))
 (segment (start 138.29 83.325) (end 138.3 83.335) (width 0.6) (layer F.Cu) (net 6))
 (segment (start 138.29 81.77) (end 138.29 83.325) (width 0.6) (layer F.Cu) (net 6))
 (segment (start 132.74 81.36) (end 133.2075 81.36) (width 0.6) (layer F.Cu) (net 5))
 (segment (start 129.65 84.45) (end 132.74 81.36) (width 0.6) (layer F.Cu) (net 5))
 (segment (start 131.08 86.93) (end 130.6 86.45) (width 0.6) (layer F.Cu) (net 3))
 (segment (start 131.08 88.95) (end 131.08 86.93) (width 0.6) (layer F.Cu) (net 3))
 (segment (start 131.08 88.145) (end 133.225 86) (width 0.6) (layer F.Cu) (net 3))
 (segment (start 131.08 88.95) (end 131.08 88.145) (width 0.6) (layer F.Cu) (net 3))
 (segment (start 124.73 80.76) (end 125.3 80.19) (width 0.6) (layer F.Cu) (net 1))
 (segment (start 122.2 80.76) (end 124.73 80.76) (width 0.6) (layer F.Cu) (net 1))
 (segment (start 126.14 79.35) (end 125.3 80.19) (width 0.6) (layer F.Cu) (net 1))
 (segment (start 129.5775 79.35) (end 126.14 79.35) (width 0.6) (layer F.Cu) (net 1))
 (segment (start 129.5775 80.9125) (end 129.63 80.965) (width 0.6) (layer F.Cu) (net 1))
 (segment (start 129.5775 79.35) (end 129.5775 80.9125) (width 0.6) (layer F.Cu) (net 1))
 (segment (start 125.3 80.19) (end 126.65 80.19) (width 0.6) (layer B.Cu) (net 1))
 (segment (start 126.22 80.19) (end 127.94 81.91) (width 0.6) (layer B.Cu) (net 1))
 (segment (start 125.3 80.19) (end 126.22 80.19) (width 0.6) (layer B.Cu) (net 1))
 (segment (start 127.94 81.91) (end 127.94 85.24) (width 0.6) (layer B.Cu) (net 1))
 (segment (start 127.94 85.24) (end 127.02 86.16) (width 0.6) (layer B.Cu) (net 1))
 (segment (start 126.25 86.16) (end 123.46 88.95) (width 0.6) (layer B.Cu) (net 1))
 (segment (start 127.02 86.16) (end 126.25 86.16) (width 0.6) (layer B.Cu) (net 1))
 (segment (start 136.1625 83.66) (end 134.62 85.2025) (width 0.6) (layer F.Cu) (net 4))
 (segment (start 134.62 87.95) (end 133.62 88.95) (width 0.6) (layer F.Cu) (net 4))
 (segment (start 134.62 85.2025) (end 134.62 87.95) (width 0.6) (layer F.Cu) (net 4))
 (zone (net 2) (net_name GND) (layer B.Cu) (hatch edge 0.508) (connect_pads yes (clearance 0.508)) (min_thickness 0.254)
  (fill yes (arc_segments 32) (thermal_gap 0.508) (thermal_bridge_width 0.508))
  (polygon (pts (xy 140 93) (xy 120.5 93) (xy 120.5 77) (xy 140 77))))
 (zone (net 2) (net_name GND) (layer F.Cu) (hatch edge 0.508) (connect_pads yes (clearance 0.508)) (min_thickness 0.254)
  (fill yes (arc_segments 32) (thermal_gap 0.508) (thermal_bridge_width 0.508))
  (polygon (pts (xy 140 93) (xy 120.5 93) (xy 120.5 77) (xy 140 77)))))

